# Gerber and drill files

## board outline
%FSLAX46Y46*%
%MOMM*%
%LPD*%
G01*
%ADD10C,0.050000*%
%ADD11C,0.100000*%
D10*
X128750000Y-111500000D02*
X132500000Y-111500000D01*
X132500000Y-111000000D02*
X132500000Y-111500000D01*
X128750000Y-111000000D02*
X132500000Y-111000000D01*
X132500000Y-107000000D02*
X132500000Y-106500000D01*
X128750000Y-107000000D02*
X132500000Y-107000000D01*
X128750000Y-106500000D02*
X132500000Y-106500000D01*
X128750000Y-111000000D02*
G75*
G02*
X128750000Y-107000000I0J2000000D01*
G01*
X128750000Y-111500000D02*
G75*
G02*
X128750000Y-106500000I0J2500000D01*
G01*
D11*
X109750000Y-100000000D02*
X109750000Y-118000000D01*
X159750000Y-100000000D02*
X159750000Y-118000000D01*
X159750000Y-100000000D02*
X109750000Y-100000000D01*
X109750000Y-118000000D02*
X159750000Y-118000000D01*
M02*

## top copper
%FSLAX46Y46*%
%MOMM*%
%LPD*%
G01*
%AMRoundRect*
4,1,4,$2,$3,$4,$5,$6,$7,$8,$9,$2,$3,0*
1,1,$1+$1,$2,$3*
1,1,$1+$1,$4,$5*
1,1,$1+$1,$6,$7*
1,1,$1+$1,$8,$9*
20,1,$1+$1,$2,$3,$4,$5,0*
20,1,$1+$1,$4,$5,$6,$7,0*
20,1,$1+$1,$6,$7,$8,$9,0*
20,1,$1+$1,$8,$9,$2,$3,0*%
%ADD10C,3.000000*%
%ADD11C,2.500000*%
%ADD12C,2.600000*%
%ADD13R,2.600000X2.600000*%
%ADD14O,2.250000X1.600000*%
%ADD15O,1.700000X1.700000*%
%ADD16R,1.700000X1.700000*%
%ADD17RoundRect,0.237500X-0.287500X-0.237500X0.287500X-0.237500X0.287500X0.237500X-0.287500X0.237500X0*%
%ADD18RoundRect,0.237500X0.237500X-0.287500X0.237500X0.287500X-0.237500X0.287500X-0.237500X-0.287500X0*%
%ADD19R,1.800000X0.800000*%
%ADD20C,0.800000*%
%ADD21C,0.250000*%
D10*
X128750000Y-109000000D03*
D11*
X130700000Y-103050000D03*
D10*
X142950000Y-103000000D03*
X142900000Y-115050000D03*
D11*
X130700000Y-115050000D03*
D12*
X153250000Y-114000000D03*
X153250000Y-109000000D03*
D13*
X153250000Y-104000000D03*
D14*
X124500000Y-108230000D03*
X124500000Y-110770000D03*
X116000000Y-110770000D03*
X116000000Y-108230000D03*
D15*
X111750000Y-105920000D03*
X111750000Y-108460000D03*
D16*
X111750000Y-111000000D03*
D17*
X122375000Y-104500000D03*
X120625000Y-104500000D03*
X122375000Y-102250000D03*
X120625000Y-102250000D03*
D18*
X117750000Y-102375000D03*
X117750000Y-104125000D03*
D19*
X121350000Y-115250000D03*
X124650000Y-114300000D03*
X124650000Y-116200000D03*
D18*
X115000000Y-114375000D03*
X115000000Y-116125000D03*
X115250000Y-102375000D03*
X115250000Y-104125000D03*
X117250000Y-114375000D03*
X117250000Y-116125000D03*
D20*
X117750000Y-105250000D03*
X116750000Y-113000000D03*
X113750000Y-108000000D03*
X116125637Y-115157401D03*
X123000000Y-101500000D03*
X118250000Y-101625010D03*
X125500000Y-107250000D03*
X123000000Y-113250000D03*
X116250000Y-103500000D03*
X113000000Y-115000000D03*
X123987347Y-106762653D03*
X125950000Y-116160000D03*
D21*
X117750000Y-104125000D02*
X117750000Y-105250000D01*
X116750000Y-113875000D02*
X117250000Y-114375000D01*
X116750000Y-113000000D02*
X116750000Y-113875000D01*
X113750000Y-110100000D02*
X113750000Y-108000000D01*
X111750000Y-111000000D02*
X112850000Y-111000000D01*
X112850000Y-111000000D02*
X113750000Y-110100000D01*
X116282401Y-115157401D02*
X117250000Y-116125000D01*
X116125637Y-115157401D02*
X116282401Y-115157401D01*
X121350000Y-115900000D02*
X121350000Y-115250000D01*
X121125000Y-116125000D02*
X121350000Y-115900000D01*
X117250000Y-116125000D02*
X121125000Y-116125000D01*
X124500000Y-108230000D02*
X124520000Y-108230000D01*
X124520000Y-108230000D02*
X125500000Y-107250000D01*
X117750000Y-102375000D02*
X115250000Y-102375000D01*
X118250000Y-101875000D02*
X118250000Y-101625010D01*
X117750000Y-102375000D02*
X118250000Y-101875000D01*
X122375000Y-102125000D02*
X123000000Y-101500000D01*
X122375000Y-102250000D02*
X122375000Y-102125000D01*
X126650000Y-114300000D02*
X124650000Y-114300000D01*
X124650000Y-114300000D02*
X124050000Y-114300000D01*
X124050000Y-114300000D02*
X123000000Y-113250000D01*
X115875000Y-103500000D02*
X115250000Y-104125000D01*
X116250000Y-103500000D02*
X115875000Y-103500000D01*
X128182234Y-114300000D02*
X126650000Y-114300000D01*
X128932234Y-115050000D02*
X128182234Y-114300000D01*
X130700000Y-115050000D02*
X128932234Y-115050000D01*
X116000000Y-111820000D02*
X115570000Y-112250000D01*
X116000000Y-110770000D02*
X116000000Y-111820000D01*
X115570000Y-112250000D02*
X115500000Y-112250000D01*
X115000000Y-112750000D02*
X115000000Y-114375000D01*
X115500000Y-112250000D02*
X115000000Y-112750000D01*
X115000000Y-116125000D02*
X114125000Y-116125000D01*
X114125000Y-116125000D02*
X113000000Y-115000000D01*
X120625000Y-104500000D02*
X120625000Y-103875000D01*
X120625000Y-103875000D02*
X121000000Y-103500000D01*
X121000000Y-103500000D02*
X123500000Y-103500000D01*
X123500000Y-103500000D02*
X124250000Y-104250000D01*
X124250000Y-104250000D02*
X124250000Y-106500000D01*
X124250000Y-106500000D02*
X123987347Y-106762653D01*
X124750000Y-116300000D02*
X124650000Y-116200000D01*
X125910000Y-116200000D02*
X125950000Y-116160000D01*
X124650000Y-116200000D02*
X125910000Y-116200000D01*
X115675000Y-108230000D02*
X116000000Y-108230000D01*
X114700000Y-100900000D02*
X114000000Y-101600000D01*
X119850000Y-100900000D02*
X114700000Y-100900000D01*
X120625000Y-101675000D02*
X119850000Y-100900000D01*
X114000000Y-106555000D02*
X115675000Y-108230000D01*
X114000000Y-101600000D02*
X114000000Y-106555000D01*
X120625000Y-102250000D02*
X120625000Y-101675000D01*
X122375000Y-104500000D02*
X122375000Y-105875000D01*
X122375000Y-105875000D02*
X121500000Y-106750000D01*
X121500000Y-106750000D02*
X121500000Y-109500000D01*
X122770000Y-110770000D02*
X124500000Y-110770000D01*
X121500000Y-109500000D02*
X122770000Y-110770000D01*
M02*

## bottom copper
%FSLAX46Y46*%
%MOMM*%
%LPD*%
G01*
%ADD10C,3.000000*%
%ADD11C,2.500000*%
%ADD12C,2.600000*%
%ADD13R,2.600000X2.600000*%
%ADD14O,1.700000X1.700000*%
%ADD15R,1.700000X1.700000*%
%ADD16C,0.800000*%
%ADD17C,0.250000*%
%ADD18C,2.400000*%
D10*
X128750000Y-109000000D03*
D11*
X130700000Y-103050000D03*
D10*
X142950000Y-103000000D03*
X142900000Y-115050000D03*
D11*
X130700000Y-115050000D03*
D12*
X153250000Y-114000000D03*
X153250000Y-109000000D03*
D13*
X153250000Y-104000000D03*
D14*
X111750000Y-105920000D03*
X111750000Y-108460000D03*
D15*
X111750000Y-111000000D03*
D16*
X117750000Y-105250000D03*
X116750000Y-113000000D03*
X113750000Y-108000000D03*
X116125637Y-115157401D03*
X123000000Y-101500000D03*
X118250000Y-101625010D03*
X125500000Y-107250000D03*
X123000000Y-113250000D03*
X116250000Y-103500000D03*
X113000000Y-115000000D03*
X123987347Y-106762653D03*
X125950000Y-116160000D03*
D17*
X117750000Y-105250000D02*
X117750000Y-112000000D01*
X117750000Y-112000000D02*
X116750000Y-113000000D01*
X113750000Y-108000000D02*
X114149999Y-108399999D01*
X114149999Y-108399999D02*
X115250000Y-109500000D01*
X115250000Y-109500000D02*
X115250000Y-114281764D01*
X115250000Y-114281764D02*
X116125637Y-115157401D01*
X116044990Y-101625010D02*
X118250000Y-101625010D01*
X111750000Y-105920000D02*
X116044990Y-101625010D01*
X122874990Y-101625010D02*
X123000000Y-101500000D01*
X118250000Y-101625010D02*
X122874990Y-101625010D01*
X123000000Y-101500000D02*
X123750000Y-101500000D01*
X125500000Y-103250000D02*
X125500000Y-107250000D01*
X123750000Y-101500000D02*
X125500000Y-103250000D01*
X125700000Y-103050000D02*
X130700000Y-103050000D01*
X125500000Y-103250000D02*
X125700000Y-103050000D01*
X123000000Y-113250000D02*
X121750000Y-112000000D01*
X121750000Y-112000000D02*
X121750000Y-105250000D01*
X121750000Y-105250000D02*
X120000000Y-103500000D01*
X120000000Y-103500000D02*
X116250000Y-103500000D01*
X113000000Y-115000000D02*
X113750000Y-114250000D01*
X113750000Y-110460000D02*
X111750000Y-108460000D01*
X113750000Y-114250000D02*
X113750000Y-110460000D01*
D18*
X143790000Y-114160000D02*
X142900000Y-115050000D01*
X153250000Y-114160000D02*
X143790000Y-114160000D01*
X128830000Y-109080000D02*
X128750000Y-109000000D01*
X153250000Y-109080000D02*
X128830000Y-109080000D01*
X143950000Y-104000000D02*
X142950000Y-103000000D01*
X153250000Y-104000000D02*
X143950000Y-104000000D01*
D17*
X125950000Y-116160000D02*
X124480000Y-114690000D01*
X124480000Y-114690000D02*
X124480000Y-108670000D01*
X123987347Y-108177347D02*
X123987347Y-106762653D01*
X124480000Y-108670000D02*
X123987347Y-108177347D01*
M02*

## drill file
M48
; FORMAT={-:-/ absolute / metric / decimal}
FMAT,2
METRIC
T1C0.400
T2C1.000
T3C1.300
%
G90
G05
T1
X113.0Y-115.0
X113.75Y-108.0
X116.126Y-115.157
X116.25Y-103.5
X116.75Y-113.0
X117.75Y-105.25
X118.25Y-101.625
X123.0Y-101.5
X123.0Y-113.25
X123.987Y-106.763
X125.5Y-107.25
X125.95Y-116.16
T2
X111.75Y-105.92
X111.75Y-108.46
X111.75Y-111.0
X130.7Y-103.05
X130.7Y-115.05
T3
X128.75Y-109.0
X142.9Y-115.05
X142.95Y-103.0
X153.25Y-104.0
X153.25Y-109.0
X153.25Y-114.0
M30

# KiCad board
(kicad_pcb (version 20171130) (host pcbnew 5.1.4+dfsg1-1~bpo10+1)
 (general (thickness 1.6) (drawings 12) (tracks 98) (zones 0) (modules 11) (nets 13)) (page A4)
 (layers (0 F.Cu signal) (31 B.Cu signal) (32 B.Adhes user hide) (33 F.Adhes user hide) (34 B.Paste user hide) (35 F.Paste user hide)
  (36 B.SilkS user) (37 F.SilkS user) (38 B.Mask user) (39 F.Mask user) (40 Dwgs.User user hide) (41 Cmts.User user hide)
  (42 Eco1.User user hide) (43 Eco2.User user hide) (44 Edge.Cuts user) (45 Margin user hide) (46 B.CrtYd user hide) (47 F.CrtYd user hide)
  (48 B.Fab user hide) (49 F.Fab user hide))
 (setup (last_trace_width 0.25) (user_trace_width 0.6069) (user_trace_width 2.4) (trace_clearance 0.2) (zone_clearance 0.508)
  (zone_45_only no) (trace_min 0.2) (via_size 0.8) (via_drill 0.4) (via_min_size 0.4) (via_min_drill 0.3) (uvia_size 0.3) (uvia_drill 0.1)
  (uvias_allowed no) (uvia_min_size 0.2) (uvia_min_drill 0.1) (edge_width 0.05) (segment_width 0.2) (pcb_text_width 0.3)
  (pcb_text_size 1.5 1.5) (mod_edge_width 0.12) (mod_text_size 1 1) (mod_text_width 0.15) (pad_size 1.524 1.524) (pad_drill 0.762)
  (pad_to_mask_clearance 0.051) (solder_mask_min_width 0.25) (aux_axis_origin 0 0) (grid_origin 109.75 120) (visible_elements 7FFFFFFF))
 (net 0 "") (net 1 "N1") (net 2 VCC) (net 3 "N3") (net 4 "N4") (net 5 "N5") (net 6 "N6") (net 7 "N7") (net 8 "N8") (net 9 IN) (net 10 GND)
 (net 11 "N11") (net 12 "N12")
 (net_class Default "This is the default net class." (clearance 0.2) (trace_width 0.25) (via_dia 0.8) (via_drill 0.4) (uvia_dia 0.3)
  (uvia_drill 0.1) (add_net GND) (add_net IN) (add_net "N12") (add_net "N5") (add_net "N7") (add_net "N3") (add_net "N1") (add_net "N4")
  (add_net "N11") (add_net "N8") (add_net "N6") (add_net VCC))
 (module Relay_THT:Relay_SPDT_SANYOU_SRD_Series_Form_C (layer F.Cu) (at 128.75 109)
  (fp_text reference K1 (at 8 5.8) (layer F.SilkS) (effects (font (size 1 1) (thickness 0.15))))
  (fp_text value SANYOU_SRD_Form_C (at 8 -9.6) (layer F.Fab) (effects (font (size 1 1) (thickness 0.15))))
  (pad 1 thru_hole circle (at 0 0 90) (size 3 3) (drill 1.3) (layers *.Cu *.Mask) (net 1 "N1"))
  (pad 5 thru_hole circle (at 1.95 -5.95 90) (size 2.5 2.5) (drill 1) (layers *.Cu *.Mask) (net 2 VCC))
  (pad 4 thru_hole circle (at 14.2 -6 90) (size 3 3) (drill 1.3) (layers *.Cu *.Mask) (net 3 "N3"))
  (pad 3 thru_hole circle (at 14.15 6.05 90) (size 3 3) (drill 1.3) (layers *.Cu *.Mask) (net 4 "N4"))
  (pad 2 thru_hole circle (at 1.95 6.05 90) (size 2.5 2.5) (drill 1) (layers *.Cu *.Mask) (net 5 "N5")))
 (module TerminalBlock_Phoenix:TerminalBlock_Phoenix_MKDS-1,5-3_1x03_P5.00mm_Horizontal (layer F.Cu) (at 153.25 104 270)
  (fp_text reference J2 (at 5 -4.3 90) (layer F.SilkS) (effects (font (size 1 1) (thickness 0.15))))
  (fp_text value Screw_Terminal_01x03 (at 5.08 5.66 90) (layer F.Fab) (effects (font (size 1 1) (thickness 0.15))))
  (pad 3 thru_hole circle (at 10 0 270) (size 2.6 2.6) (drill 1.3) (layers *.Cu *.Mask) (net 4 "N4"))
  (pad 2 thru_hole circle (at 5 0 270) (size 2.6 2.6) (drill 1.3) (layers *.Cu *.Mask) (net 1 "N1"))
  (pad 1 thru_hole rect (at 0 0 270) (size 2.6 2.6) (drill 1.3) (layers *.Cu *.Mask) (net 3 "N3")))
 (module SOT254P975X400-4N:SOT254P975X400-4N (layer F.Cu) (at 120.25 109.5)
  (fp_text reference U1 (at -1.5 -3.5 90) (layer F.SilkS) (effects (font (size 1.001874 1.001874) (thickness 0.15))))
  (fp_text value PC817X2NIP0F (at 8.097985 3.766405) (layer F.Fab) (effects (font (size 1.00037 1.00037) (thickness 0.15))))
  (pad 4 smd oval (at 4.25 -1.27) (size 2.25 1.6) (layers F.Cu F.Paste F.Mask) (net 2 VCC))
  (pad 3 smd oval (at 4.25 1.27) (size 2.25 1.6) (layers F.Cu F.Paste F.Mask) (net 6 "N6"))
  (pad 2 smd oval (at -4.25 1.27) (size 2.25 1.6) (layers F.Cu F.Paste F.Mask) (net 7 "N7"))
  (pad 1 smd oval (at -4.25 -1.27) (size 2.25 1.6) (layers F.Cu F.Paste F.Mask) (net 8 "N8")))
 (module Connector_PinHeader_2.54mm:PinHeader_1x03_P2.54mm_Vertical (layer F.Cu) (at 111.75 111 180)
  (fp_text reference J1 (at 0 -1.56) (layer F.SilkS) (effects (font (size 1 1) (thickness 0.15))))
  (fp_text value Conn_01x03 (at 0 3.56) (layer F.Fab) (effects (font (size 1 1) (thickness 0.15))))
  (pad 3 thru_hole oval (at 0 5.08 180) (size 1.7 1.7) (drill 1) (layers *.Cu *.Mask) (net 2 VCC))
  (pad 2 thru_hole oval (at 0 2.54 180) (size 1.7 1.7) (drill 1) (layers *.Cu *.Mask) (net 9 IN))
  (pad 1 thru_hole rect (at 0 0 180) (size 1.7 1.7) (drill 1) (layers *.Cu *.Mask) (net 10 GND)))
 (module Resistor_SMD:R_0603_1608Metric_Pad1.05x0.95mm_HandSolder (layer F.Cu) (at 121.5 104.5)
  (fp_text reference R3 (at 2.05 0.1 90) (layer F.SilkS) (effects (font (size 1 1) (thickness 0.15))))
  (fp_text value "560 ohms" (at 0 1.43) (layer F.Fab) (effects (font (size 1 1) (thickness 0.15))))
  (pad 2 smd roundrect (at 0.875 0) (size 1.05 0.95) (layers F.Cu F.Paste F.Mask) (roundrect_rratio 0.25) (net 6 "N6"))
  (pad 1 smd roundrect (at -0.875 0) (size 1.05 0.95) (layers F.Cu F.Paste F.Mask) (roundrect_rratio 0.25) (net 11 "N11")))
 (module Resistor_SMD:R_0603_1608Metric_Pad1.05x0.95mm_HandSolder (layer F.Cu) (at 121.5 102.25)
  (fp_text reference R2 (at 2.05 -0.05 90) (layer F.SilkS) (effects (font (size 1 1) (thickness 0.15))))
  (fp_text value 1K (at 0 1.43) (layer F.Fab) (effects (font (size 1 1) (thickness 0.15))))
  (pad 2 smd roundrect (at 0.875 0) (size 1.05 0.95) (layers F.Cu F.Paste F.Mask) (roundrect_rratio 0.25) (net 2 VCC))
  (pad 1 smd roundrect (at -0.875 0) (size 1.05 0.95) (layers F.Cu F.Paste F.Mask) (roundrect_rratio 0.25) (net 8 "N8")))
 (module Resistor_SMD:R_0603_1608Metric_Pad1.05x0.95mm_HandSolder (layer F.Cu) (at 117.75 103.25 90)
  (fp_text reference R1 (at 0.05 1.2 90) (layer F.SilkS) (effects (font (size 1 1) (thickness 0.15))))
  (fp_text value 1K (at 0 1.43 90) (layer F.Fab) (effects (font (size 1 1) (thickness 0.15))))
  (pad 2 smd roundrect (at 0.875 0 90) (size 1.05 0.95) (layers F.Cu F.Paste F.Mask) (roundrect_rratio 0.25) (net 2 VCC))
  (pad 1 smd roundrect (at -0.875 0 90) (size 1.05 0.95) (layers F.Cu F.Paste F.Mask) (roundrect_rratio 0.25) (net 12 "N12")))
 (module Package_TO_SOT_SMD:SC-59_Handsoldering (layer F.Cu) (at 123 115.25 180)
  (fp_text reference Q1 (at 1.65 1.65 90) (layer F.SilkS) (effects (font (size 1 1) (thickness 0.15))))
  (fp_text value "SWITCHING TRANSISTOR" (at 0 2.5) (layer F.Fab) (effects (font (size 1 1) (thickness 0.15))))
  (pad 3 smd rect (at 1.65 0 180) (size 1.8 0.8) (layers F.Cu F.Paste F.Mask) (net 10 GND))
  (pad 2 smd rect (at -1.65 0.95 180) (size 1.8 0.8) (layers F.Cu F.Paste F.Mask) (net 5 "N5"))
  (pad 1 smd rect (at -1.65 -0.95 180) (size 1.8 0.8) (layers F.Cu F.Paste F.Mask) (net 11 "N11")))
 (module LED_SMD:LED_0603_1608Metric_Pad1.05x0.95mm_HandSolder (layer F.Cu) (at 115 115.25 90)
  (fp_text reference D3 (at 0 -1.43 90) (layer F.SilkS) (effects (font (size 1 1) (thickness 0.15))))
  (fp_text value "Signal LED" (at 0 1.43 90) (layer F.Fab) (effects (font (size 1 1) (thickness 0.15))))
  (pad 2 smd roundrect (at 0.875 0 90) (size 1.05 0.95) (layers F.Cu F.Paste F.Mask) (roundrect_rratio 0.25) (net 7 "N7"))
  (pad 1 smd roundrect (at -0.875 0 90) (size 1.05 0.95) (layers F.Cu F.Paste F.Mask) (roundrect_rratio 0.25) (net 9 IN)))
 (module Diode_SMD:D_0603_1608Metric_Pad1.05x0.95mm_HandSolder (layer F.Cu) (at 115.25 103.25 90)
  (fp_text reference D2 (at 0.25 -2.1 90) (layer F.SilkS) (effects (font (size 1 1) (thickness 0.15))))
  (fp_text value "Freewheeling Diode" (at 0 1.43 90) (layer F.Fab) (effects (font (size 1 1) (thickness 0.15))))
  (pad 2 smd roundrect (at 0.875 0 90) (size 1.05 0.95) (layers F.Cu F.Paste F.Mask) (roundrect_rratio 0.25) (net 2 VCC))
  (pad 1 smd roundrect (at -0.875 0 90) (size 1.05 0.95) (layers F.Cu F.Paste F.Mask) (roundrect_rratio 0.25) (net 5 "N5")))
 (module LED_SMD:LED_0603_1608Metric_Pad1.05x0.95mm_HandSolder (layer F.Cu) (at 117.25 115.25 90)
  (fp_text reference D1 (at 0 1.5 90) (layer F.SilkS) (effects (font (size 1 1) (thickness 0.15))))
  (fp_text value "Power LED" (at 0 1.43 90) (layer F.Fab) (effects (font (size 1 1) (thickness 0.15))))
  (pad 2 smd roundrect (at 0.875 0 90) (size 1.05 0.95) (layers F.Cu F.Paste F.Mask) (roundrect_rratio 0.25) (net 12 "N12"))
  (pad 1 smd roundrect (at -0.875 0 90) (size 1.05 0.95) (layers F.Cu F.Paste F.Mask) (roundrect_rratio 0.25) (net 10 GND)))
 (gr_line (start 128.75 111.5) (end 132.5 111.5) (layer Edge.Cuts) (width 0.05))
 (gr_line (start 132.5 111) (end 132.5 111.5) (layer Edge.Cuts) (width 0.05))
 (gr_line (start 128.75 111) (end 132.5 111) (layer Edge.Cuts) (width 0.05))
 (gr_line (start 132.5 107) (end 132.5 106.5) (layer Edge.Cuts) (width 0.05))
 (gr_line (start 128.75 107) (end 132.5 107) (layer Edge.Cuts) (width 0.05))
 (gr_line (start 128.75 106.5) (end 132.5 106.5) (layer Edge.Cuts) (width 0.05))
 (gr_arc (start 128.75 109) (end 128.75 107) (angle -180) (layer Edge.Cuts) (width 0.05))
 (gr_arc (start 128.75 109) (end 128.75 106.5) (angle -180) (layer Edge.Cuts) (width 0.05))
 (gr_line (start 109.75 100) (end 109.75 118) (layer Edge.Cuts) (width 0.1))
 (gr_line (start 159.75 100) (end 159.75 118) (layer Edge.Cuts) (width 0.1))
 (gr_line (start 159.75 100) (end 109.75 100) (layer Edge.Cuts) (width 0.1))
 (gr_line (start 109.75 118) (end 159.75 118) (layer Edge.Cuts) (width 0.1))
 (via (at 117.75 105.25) (size 0.8) (drill 0.4) (layers F.Cu B.Cu) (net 12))
 (segment (start 117.75 104.125) (end 117.75 105.25) (width 0.25) (layer F.Cu) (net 12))
 (via (at 116.75 113) (size 0.8) (drill 0.4) (layers F.Cu B.Cu) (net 12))
 (segment (start 117.75 105.25) (end 117.75 112) (width 0.25) (layer B.Cu) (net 12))
 (segment (start 117.75 112) (end 116.75 113) (width 0.25) (layer B.Cu) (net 12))
 (segment (start 116.75 113.875) (end 117.25 114.375) (width 0.25) (layer F.Cu) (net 12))
 (segment (start 116.75 113) (end 116.75 113.875) (width 0.25) (layer F.Cu) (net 12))
 (via (at 113.75 108) (size 0.8) (drill 0.4) (layers F.Cu B.Cu) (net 10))
 (segment (start 113.75 110.1) (end 113.75 108) (width 0.25) (layer F.Cu) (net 10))
 (segment (start 111.75 111) (end 112.85 111) (width 0.25) (layer F.Cu) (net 10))
 (segment (start 112.85 111) (end 113.75 110.1) (width 0.25) (layer F.Cu) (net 10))
 (segment (start 113.75 108) (end 114.149999 108.399999) (width 0.25) (layer B.Cu) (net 10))
 (segment (start 114.149999 108.399999) (end 115.25 109.5) (width 0.25) (layer B.Cu) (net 10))
 (via (at 116.125637 115.157401) (size 0.8) (drill 0.4) (layers F.Cu B.Cu) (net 10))
 (segment (start 115.25 109.5) (end 115.25 114.281764) (width 0.25) (layer B.Cu) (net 10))
 (segment (start 115.25 114.281764) (end 116.125637 115.157401) (width 0.25) (layer B.Cu) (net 10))
 (segment (start 116.282401 115.157401) (end 117.25 116.125) (width 0.25) (layer F.Cu) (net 10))
 (segment (start 116.125637 115.157401) (end 116.282401 115.157401) (width 0.25) (layer F.Cu) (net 10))
 (segment (start 121.35 115.9) (end 121.35 115.25) (width 0.25) (layer F.Cu) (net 10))
 (segment (start 121.125 116.125) (end 121.35 115.9) (width 0.25) (layer F.Cu) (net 10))
 (segment (start 117.25 116.125) (end 121.125 116.125) (width 0.25) (layer F.Cu) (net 10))
 (segment (start 124.5 108.23) (end 124.52 108.23) (width 0.25) (layer F.Cu) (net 2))
 (segment (start 124.52 108.23) (end 125.5 107.25) (width 0.25) (layer F.Cu) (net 2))
 (via (at 123 101.5) (size 0.8) (drill 0.4) (layers F.Cu B.Cu) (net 2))
 (segment (start 117.75 102.375) (end 115.25 102.375) (width 0.25) (layer F.Cu) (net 2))
 (segment (start 118.25 101.875) (end 118.25 101.62501) (width 0.25) (layer F.Cu) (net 2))
 (segment (start 117.75 102.375) (end 118.25 101.875) (width 0.25) (layer F.Cu) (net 2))
 (segment (start 122.375 102.125) (end 123 101.5) (width 0.25) (layer F.Cu) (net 2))
 (segment (start 122.375 102.25) (end 122.375 102.125) (width 0.25) (layer F.Cu) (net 2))
 (via (at 118.25 101.62501) (size 0.8) (drill 0.4) (layers F.Cu B.Cu) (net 2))
 (via (at 125.5 107.25) (size 0.8) (drill 0.4) (layers F.Cu B.Cu) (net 2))
 (segment (start 116.04499 101.62501) (end 118.25 101.62501) (width 0.25) (layer B.Cu) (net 2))
 (segment (start 111.75 105.92) (end 116.04499 101.62501) (width 0.25) (layer B.Cu) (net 2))
 (segment (start 122.87499 101.62501) (end 123 101.5) (width 0.25) (layer B.Cu) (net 2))
 (segment (start 118.25 101.62501) (end 122.87499 101.62501) (width 0.25) (layer B.Cu) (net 2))
 (segment (start 123 101.5) (end 123.75 101.5) (width 0.25) (layer B.Cu) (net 2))
 (segment (start 125.5 103.25) (end 125.5 107.25) (width 0.25) (layer B.Cu) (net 2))
 (segment (start 123.75 101.5) (end 125.5 103.25) (width 0.25) (layer B.Cu) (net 2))
 (segment (start 125.7 103.05) (end 130.7 103.05) (width 0.25) (layer B.Cu) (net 2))
 (segment (start 125.5 103.25) (end 125.7 103.05) (width 0.25) (layer B.Cu) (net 2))
 (segment (start 126.65 114.3) (end 124.65 114.3) (width 0.25) (layer F.Cu) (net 5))
 (via (at 123 113.25) (size 0.8) (drill 0.4) (layers F.Cu B.Cu) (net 5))
 (segment (start 124.65 114.3) (end 124.05 114.3) (width 0.25) (layer F.Cu) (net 5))
 (segment (start 124.05 114.3) (end 123 113.25) (width 0.25) (layer F.Cu) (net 5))
 (segment (start 123 113.25) (end 121.75 112) (width 0.25) (layer B.Cu) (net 5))
 (segment (start 121.75 112) (end 121.75 105.25) (width 0.25) (layer B.Cu) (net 5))
 (via (at 116.25 103.5) (size 0.8) (drill 0.4) (layers F.Cu B.Cu) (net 5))
 (segment (start 121.75 105.25) (end 120 103.5) (width 0.25) (layer B.Cu) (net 5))
 (segment (start 120 103.5) (end 116.25 103.5) (width 0.25) (layer B.Cu) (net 5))
 (segment (start 115.875 103.5) (end 115.25 104.125) (width 0.25) (layer F.Cu) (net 5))
 (segment (start 116.25 103.5) (end 115.875 103.5) (width 0.25) (layer F.Cu) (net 5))
 (segment (start 128.182234 114.3) (end 126.65 114.3) (width 0.25) (layer F.Cu) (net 5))
 (segment (start 128.932234 115.05) (end 128.182234 114.3) (width 0.25) (layer F.Cu) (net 5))
 (segment (start 130.7 115.05) (end 128.932234 115.05) (width 0.25) (layer F.Cu) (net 5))
 (segment (start 116 111.82) (end 115.57 112.25) (width 0.25) (layer F.Cu) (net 7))
 (segment (start 116 110.77) (end 116 111.82) (width 0.25) (layer F.Cu) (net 7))
 (segment (start 115.57 112.25) (end 115.5 112.25) (width 0.25) (layer F.Cu) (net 7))
 (segment (start 115 112.75) (end 115 114.375) (width 0.25) (layer F.Cu) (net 7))
 (segment (start 115.5 112.25) (end 115 112.75) (width 0.25) (layer F.Cu) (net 7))
 (segment (start 115 116.125) (end 114.125 116.125) (width 0.25) (layer F.Cu) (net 9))
 (via (at 113 115) (size 0.8) (drill 0.4) (layers F.Cu B.Cu) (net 9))
 (segment (start 114.125 116.125) (end 113 115) (width 0.25) (layer F.Cu) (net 9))
 (segment (start 113 115) (end 113.75 114.25) (width 0.25) (layer B.Cu) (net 9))
 (segment (start 113.75 110.46) (end 111.75 108.46) (width 0.25) (layer B.Cu) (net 9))
 (segment (start 113.75 114.25) (end 113.75 110.46) (width 0.25) (layer B.Cu) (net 9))
 (segment (start 143.79 114.16) (end 142.9 115.05) (width 2.4) (layer B.Cu) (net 4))
 (segment (start 153.25 114.16) (end 143.79 114.16) (width 2.4) (layer B.Cu) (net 4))
 (segment (start 128.83 109.08) (end 128.75 109) (width 2.4) (layer B.Cu) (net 1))
 (segment (start 153.25 109.08) (end 128.83 109.08) (width 2.4) (layer B.Cu) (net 1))
 (segment (start 143.95 104) (end 142.95 103) (width 2.4) (layer B.Cu) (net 3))
 (segment (start 153.25 104) (end 143.95 104) (width 2.4) (layer B.Cu) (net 3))
 (segment (start 120.625 104.5) (end 120.625 103.875) (width 0.25) (layer F.Cu) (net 11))
 (segment (start 120.625 103.875) (end 121 103.5) (width 0.25) (layer F.Cu) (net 11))
 (segment (start 121 103.5) (end 123.5 103.5) (width 0.25) (layer F.Cu) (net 11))
 (segment (start 123.5 103.5) (end 124.25 104.25) (width 0.25) (layer F.Cu) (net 11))
 (via (at 123.987347 106.762653) (size 0.8) (drill 0.4) (layers F.Cu B.Cu) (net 11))
 (segment (start 124.25 104.25) (end 124.25 106.5) (width 0.25) (layer F.Cu) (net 11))
 (segment (start 124.25 106.5) (end 123.987347 106.762653) (width 0.25) (layer F.Cu) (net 11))
 (via (at 125.95 116.16) (size 0.8) (drill 0.4) (layers F.Cu B.Cu) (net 11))
 (segment (start 124.75 116.3) (end 124.65 116.2) (width 0.25) (layer F.Cu) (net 11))
 (segment (start 125.95 116.16) (end 124.48 114.69) (width 0.25) (layer B.Cu) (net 11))
 (segment (start 124.48 114.69) (end 124.48 108.67) (width 0.25) (layer B.Cu) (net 11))
 (segment (start 123.987347 108.177347) (end 123.987347 106.762653) (width 0.25) (layer B.Cu) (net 11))
 (segment (start 124.48 108.67) (end 123.987347 108.177347) (width 0.25) (layer B.Cu) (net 11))
 (segment (start 125.91 116.2) (end 125.95 116.16) (width 0.25) (layer F.Cu) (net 11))
 (segment (start 124.65 116.2) (end 125.91 116.2) (width 0.25) (layer F.Cu) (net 11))
 (segment (start 115.675 108.23) (end 116 108.23) (width 0.25) (layer F.Cu) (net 8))
 (segment (start 114.7 100.9) (end 114 101.6) (width 0.25) (layer F.Cu) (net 8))
 (segment (start 119.85 100.9) (end 114.7 100.9) (width 0.25) (layer F.Cu) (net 8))
 (segment (start 120.625 101.675) (end 119.85 100.9) (width 0.25) (layer F.Cu) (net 8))
 (segment (start 114 106.555) (end 115.675 108.23) (width 0.25) (layer F.Cu) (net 8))
 (segment (start 114 101.6) (end 114 106.555) (width 0.25) (layer F.Cu) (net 8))
 (segment (start 120.625 102.25) (end 120.625 101.675) (width 0.25) (layer F.Cu) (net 8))
 (segment (start 122.375 104.5) (end 122.375 105.875) (width 0.25) (layer F.Cu) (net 6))
 (segment (start 122.375 105.875) (end 121.5 106.75) (width 0.25) (layer F.Cu) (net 6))
 (segment (start 121.5 106.75) (end 121.5 109.5) (width 0.25) (layer F.Cu) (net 6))
 (segment (start 122.77 110.77) (end 124.5 110.77) (width 0.25) (layer F.Cu) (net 6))
 (segment (start 121.5 109.5) (end 122.77 110.77) (width 0.25) (layer F.Cu) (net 6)))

